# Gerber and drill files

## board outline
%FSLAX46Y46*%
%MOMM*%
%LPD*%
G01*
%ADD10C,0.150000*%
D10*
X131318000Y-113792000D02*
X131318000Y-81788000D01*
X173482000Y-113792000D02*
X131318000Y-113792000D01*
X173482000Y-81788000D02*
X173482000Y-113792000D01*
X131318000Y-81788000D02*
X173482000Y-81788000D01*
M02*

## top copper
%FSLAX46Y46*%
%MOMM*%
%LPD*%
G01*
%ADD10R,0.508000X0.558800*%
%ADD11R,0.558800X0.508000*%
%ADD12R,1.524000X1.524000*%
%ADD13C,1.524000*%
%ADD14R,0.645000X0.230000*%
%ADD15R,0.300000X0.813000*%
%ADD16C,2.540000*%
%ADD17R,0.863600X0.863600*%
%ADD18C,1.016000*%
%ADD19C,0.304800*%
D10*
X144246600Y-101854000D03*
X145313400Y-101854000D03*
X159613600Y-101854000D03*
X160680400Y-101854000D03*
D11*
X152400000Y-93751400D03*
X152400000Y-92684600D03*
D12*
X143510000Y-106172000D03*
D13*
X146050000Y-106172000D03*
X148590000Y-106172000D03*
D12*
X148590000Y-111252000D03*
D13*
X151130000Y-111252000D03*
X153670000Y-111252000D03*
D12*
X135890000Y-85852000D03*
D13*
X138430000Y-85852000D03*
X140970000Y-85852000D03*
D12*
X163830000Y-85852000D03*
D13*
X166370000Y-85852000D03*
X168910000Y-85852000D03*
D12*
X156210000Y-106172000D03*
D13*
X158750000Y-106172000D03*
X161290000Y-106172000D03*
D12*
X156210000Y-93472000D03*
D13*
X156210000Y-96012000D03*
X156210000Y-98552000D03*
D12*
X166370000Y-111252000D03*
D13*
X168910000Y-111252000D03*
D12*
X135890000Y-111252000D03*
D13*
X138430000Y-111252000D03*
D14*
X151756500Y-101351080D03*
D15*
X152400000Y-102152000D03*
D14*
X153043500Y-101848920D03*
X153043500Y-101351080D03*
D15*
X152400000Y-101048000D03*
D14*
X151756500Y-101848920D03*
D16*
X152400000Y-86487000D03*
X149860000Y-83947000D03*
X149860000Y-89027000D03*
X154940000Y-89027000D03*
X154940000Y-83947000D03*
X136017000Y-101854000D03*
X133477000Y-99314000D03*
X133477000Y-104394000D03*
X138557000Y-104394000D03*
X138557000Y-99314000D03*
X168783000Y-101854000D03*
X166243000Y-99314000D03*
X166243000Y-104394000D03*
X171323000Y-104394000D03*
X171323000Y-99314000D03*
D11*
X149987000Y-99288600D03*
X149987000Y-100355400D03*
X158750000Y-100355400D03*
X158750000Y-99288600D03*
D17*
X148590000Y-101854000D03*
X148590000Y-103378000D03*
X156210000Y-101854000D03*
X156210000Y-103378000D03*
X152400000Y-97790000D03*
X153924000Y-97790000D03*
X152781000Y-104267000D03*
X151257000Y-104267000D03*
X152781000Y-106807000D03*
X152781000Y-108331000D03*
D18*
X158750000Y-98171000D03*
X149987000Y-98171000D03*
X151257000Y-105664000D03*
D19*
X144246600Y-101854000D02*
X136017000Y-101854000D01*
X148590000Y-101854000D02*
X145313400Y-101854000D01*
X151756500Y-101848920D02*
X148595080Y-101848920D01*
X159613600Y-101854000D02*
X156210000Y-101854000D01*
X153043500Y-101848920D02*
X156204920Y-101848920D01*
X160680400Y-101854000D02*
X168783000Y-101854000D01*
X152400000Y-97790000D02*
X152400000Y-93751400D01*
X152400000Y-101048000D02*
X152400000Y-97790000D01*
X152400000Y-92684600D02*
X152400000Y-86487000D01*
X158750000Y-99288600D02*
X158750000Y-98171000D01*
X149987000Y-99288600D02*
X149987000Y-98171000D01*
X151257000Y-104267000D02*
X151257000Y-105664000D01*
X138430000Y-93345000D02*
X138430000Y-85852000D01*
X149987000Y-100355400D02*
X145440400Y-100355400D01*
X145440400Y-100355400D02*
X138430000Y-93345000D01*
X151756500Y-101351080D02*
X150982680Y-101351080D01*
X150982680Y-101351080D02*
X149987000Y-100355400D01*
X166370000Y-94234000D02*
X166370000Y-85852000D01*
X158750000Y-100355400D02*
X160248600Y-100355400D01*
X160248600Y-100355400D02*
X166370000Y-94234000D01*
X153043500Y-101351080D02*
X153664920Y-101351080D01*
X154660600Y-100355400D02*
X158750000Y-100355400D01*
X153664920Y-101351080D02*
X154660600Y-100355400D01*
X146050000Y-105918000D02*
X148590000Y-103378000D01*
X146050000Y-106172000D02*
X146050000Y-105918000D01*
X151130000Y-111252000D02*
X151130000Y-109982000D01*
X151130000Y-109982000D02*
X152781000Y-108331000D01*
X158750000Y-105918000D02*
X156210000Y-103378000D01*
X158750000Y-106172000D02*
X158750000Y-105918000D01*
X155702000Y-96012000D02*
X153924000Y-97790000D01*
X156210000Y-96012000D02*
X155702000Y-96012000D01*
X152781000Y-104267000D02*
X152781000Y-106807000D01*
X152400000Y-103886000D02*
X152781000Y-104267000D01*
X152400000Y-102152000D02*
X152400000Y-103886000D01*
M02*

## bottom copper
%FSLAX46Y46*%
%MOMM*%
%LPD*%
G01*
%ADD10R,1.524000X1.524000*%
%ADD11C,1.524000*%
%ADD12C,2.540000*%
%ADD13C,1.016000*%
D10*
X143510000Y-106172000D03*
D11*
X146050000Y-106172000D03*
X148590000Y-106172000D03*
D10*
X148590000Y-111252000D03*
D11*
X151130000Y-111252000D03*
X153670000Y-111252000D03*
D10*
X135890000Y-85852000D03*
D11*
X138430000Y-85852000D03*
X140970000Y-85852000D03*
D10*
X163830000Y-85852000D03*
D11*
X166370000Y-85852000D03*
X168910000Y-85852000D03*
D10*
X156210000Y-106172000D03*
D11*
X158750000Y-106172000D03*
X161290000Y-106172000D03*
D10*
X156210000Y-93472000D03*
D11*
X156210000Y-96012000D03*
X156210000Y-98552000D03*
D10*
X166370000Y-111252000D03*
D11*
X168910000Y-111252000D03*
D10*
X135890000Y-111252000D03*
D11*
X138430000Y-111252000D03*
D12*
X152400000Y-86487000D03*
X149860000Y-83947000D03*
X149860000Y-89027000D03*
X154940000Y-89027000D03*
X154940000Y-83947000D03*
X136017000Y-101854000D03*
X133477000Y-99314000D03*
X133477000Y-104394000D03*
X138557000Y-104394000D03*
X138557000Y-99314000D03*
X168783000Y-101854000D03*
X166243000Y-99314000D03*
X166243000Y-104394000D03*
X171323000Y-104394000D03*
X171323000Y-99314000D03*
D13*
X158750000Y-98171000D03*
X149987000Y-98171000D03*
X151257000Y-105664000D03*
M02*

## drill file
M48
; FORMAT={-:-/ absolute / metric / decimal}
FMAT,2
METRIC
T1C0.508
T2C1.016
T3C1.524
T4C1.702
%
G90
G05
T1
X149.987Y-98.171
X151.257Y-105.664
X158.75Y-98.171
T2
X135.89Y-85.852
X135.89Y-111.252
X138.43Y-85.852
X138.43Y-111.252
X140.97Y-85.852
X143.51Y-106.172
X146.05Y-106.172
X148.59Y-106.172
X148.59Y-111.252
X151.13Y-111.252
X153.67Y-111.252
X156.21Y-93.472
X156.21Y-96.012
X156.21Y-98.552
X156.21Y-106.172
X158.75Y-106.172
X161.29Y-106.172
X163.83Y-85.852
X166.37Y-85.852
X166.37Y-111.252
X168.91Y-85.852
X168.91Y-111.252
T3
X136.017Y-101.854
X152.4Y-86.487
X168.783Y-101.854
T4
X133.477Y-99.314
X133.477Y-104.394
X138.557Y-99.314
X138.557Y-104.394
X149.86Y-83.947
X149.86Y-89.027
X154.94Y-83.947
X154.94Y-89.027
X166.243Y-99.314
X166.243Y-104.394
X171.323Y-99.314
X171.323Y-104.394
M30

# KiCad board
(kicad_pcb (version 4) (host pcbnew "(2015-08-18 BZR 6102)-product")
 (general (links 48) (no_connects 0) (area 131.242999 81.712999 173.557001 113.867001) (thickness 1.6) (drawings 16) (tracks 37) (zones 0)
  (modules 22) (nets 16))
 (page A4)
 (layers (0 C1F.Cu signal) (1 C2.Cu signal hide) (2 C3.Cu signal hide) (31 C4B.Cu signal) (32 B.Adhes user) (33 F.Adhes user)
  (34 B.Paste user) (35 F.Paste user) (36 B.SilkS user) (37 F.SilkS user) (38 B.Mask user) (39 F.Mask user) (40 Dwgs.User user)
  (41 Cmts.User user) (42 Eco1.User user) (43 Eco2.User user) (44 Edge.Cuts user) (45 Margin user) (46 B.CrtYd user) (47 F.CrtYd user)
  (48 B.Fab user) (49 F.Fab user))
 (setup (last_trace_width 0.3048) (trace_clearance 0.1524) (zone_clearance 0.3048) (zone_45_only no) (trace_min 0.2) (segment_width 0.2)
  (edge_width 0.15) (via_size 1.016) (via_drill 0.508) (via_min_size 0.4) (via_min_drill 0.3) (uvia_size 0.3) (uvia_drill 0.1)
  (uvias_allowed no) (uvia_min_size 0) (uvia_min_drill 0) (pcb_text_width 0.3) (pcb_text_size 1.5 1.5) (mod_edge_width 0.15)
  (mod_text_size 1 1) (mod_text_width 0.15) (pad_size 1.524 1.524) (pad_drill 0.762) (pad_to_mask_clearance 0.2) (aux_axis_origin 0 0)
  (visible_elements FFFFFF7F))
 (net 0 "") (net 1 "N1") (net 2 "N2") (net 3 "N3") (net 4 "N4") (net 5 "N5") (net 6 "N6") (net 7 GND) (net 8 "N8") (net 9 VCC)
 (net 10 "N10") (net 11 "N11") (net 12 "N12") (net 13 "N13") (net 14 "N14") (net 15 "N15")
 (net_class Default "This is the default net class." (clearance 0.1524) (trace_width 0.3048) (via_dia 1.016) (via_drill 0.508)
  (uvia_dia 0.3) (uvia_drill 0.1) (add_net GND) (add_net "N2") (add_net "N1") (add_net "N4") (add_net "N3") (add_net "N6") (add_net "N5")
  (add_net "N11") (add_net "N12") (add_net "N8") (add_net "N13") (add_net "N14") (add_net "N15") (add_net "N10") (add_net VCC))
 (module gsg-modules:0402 (layer C1F.Cu) (at 144.78 101.854 180) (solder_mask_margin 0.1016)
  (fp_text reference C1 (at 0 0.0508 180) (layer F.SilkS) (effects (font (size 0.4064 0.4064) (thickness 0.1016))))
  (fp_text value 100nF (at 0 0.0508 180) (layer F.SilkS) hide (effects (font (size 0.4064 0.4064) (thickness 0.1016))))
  (pad 2 smd rect (at 0.5334 0 180) (size 0.508 0.5588) (layers C1F.Cu F.Paste F.Mask) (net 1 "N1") (solder_mask_margin 0.1016))
  (pad 1 smd rect (at -0.5334 0 180) (size 0.508 0.5588) (layers C1F.Cu F.Paste F.Mask) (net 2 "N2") (solder_mask_margin 0.1016)))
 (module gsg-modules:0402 (layer C1F.Cu) (at 160.147 101.854 180) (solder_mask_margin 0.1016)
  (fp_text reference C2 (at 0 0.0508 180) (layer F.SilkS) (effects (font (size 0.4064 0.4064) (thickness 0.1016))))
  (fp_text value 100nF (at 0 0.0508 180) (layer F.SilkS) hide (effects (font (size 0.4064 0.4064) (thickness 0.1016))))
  (pad 2 smd rect (at 0.5334 0 180) (size 0.508 0.5588) (layers C1F.Cu F.Paste F.Mask) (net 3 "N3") (solder_mask_margin 0.1016))
  (pad 1 smd rect (at -0.5334 0 180) (size 0.508 0.5588) (layers C1F.Cu F.Paste F.Mask) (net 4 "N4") (solder_mask_margin 0.1016)))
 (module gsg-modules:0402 (layer C1F.Cu) (at 152.4 93.218 270) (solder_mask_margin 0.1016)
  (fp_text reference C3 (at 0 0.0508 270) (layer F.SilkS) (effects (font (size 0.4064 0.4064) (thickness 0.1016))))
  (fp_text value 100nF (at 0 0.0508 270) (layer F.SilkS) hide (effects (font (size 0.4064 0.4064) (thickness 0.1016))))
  (pad 2 smd rect (at 0.5334 0 270) (size 0.508 0.5588) (layers C1F.Cu F.Paste F.Mask) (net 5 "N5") (solder_mask_margin 0.1016))
  (pad 1 smd rect (at -0.5334 0 270) (size 0.508 0.5588) (layers C1F.Cu F.Paste F.Mask) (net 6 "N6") (solder_mask_margin 0.1016)))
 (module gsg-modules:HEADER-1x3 (layer C1F.Cu) (at 146.05 106.172)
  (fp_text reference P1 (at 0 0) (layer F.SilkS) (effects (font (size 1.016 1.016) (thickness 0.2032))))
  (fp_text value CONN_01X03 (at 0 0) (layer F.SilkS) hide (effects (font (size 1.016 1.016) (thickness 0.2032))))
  (pad 1 thru_hole rect (at -2.54 0) (size 1.524 1.524) (drill 1.016) (layers *.Cu *.Mask F.SilkS) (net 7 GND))
  (pad 2 thru_hole circle (at 0 0) (size 1.524 1.524) (drill 1.016) (layers *.Cu *.Mask F.SilkS) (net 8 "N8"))
  (pad 3 thru_hole circle (at 2.54 0) (size 1.524 1.524) (drill 1.016) (layers *.Cu *.Mask F.SilkS) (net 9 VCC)))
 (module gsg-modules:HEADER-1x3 (layer C1F.Cu) (at 151.13 111.252)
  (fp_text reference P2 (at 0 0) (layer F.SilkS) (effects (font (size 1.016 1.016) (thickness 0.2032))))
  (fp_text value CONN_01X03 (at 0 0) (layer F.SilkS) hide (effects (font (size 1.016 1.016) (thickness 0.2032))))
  (pad 1 thru_hole rect (at -2.54 0) (size 1.524 1.524) (drill 1.016) (layers *.Cu *.Mask F.SilkS) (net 7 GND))
  (pad 2 thru_hole circle (at 0 0) (size 1.524 1.524) (drill 1.016) (layers *.Cu *.Mask F.SilkS) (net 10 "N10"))
  (pad 3 thru_hole circle (at 2.54 0) (size 1.524 1.524) (drill 1.016) (layers *.Cu *.Mask F.SilkS) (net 9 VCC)))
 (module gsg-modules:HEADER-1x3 (layer C1F.Cu) (at 138.43 85.852)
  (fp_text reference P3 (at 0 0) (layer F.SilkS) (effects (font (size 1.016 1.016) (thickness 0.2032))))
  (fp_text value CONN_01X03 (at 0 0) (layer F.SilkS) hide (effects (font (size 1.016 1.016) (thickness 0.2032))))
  (pad 1 thru_hole rect (at -2.54 0) (size 1.524 1.524) (drill 1.016) (layers *.Cu *.Mask F.SilkS) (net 7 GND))
  (pad 2 thru_hole circle (at 0 0) (size 1.524 1.524) (drill 1.016) (layers *.Cu *.Mask F.SilkS) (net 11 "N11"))
  (pad 3 thru_hole circle (at 2.54 0) (size 1.524 1.524) (drill 1.016) (layers *.Cu *.Mask F.SilkS) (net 9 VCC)))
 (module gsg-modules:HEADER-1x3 (layer C1F.Cu) (at 166.37 85.852)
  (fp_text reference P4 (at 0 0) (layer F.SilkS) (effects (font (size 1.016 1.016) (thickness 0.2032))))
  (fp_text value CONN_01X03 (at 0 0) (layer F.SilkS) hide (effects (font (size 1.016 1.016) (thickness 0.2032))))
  (pad 1 thru_hole rect (at -2.54 0) (size 1.524 1.524) (drill 1.016) (layers *.Cu *.Mask F.SilkS) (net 7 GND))
  (pad 2 thru_hole circle (at 0 0) (size 1.524 1.524) (drill 1.016) (layers *.Cu *.Mask F.SilkS) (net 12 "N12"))
  (pad 3 thru_hole circle (at 2.54 0) (size 1.524 1.524) (drill 1.016) (layers *.Cu *.Mask F.SilkS) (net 9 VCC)))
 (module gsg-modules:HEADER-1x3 (layer C1F.Cu) (at 158.75 106.172)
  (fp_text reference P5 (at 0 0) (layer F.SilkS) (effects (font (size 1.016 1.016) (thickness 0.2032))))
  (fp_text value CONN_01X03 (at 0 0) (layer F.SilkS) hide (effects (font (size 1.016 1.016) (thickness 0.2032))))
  (pad 1 thru_hole rect (at -2.54 0) (size 1.524 1.524) (drill 1.016) (layers *.Cu *.Mask F.SilkS) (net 7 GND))
  (pad 2 thru_hole circle (at 0 0) (size 1.524 1.524) (drill 1.016) (layers *.Cu *.Mask F.SilkS) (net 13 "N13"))
  (pad 3 thru_hole circle (at 2.54 0) (size 1.524 1.524) (drill 1.016) (layers *.Cu *.Mask F.SilkS) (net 9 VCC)))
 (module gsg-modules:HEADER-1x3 (layer C1F.Cu) (at 156.21 96.012 270)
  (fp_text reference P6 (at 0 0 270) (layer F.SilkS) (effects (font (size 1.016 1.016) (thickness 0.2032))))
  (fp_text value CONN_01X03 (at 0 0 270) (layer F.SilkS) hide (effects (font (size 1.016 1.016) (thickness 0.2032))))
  (pad 1 thru_hole rect (at -2.54 0 270) (size 1.524 1.524) (drill 1.016) (layers *.Cu *.Mask F.SilkS) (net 7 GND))
  (pad 2 thru_hole circle (at 0 0 270) (size 1.524 1.524) (drill 1.016) (layers *.Cu *.Mask F.SilkS) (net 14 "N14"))
  (pad 3 thru_hole circle (at 2.54 0 270) (size 1.524 1.524) (drill 1.016) (layers *.Cu *.Mask F.SilkS) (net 9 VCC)))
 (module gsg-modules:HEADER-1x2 (layer C1F.Cu) (at 167.64 111.252)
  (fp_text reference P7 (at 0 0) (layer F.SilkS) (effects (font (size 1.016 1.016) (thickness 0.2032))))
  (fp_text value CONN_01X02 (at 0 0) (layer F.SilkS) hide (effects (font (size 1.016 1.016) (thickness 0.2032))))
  (pad 1 thru_hole rect (at -1.27 0) (size 1.524 1.524) (drill 1.016) (layers *.Cu *.Mask F.SilkS) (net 9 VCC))
  (pad 2 thru_hole circle (at 1.27 0) (size 1.524 1.524) (drill 1.016) (layers *.Cu *.Mask F.SilkS) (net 9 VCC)))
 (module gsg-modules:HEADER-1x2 (layer C1F.Cu) (at 137.16 111.252)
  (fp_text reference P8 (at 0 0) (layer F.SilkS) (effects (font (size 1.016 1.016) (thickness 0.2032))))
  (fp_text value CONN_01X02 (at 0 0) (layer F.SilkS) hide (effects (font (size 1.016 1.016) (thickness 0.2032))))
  (pad 1 thru_hole rect (at -1.27 0) (size 1.524 1.524) (drill 1.016) (layers *.Cu *.Mask F.SilkS) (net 7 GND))
  (pad 2 thru_hole circle (at 1.27 0) (size 1.524 1.524) (drill 1.016) (layers *.Cu *.Mask F.SilkS) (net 7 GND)))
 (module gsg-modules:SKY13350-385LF (layer C1F.Cu) (at 152.4 101.6) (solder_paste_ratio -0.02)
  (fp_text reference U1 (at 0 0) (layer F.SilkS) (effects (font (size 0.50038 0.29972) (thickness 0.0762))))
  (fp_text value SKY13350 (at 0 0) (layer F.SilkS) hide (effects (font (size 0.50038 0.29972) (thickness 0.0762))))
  (pad 1 smd rect (at -0.6435 -0.24892) (size 0.645 0.23) (layers C1F.Cu F.Paste F.Mask) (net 11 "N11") (die_length -2147.483648))
  (pad 3 smd rect (at 0 0.552) (size 0.3 0.813) (layers C1F.Cu F.Paste F.Mask) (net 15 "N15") (die_length -2147.483648))
  (pad 4 smd rect (at 0.6435 0.24892) (size 0.645 0.23) (layers C1F.Cu F.Paste F.Mask) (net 3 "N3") (die_length 0.0508))
  (pad 5 smd rect (at 0.6435 -0.24892) (size 0.645 0.23) (layers C1F.Cu F.Paste F.Mask) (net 12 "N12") (die_length 10.53846))
  (pad 6 smd rect (at 0 -0.552) (size 0.3 0.813) (layers C1F.Cu F.Paste F.Mask) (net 5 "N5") (die_length -2147.483648))
  (pad 2 smd rect (at -0.6435 0.24892) (size 0.645 0.23) (layers C1F.Cu F.Paste F.Mask) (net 2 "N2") (die_length -2147.483648)))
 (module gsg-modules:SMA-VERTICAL (layer C1F.Cu) (at 152.4 86.487)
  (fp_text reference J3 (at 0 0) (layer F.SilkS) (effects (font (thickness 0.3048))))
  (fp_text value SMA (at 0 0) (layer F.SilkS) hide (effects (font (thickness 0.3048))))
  (pad 1 thru_hole circle (at 0 0) (size 2.54 2.54) (drill 1.524) (layers *.Cu *.Mask F.SilkS) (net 6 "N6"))
  (pad 2 thru_hole circle (at -2.54 -2.54) (size 2.54 2.54) (drill 1.7018) (layers *.Cu *.Mask F.SilkS) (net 7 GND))
  (pad 2 thru_hole circle (at -2.54 2.54) (size 2.54 2.54) (drill 1.7018) (layers *.Cu *.Mask F.SilkS) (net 7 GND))
  (pad 2 thru_hole circle (at 2.54 2.54) (size 2.54 2.54) (drill 1.7018) (layers *.Cu *.Mask F.SilkS) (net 7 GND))
  (pad 2 thru_hole circle (at 2.54 -2.54) (size 2.54 2.54) (drill 1.7018) (layers *.Cu *.Mask F.SilkS) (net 7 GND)))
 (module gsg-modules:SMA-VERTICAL (layer C1F.Cu) (at 136.017 101.854)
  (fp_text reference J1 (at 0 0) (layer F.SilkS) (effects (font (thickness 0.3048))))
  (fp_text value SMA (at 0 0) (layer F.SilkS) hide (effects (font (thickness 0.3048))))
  (pad 1 thru_hole circle (at 0 0) (size 2.54 2.54) (drill 1.524) (layers *.Cu *.Mask F.SilkS) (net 1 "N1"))
  (pad 2 thru_hole circle (at -2.54 -2.54) (size 2.54 2.54) (drill 1.7018) (layers *.Cu *.Mask F.SilkS) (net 7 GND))
  (pad 2 thru_hole circle (at -2.54 2.54) (size 2.54 2.54) (drill 1.7018) (layers *.Cu *.Mask F.SilkS) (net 7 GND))
  (pad 2 thru_hole circle (at 2.54 2.54) (size 2.54 2.54) (drill 1.7018) (layers *.Cu *.Mask F.SilkS) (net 7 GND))
  (pad 2 thru_hole circle (at 2.54 -2.54) (size 2.54 2.54) (drill 1.7018) (layers *.Cu *.Mask F.SilkS) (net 7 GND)))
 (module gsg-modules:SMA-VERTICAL (layer C1F.Cu) (at 168.783 101.854)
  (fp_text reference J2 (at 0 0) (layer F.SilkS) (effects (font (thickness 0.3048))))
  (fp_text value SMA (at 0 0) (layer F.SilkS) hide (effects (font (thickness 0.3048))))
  (pad 1 thru_hole circle (at 0 0) (size 2.54 2.54) (drill 1.524) (layers *.Cu *.Mask F.SilkS) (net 4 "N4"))
  (pad 2 thru_hole circle (at -2.54 -2.54) (size 2.54 2.54) (drill 1.7018) (layers *.Cu *.Mask F.SilkS) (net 7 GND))
  (pad 2 thru_hole circle (at -2.54 2.54) (size 2.54 2.54) (drill 1.7018) (layers *.Cu *.Mask F.SilkS) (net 7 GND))
  (pad 2 thru_hole circle (at 2.54 2.54) (size 2.54 2.54) (drill 1.7018) (layers *.Cu *.Mask F.SilkS) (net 7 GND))
  (pad 2 thru_hole circle (at 2.54 -2.54) (size 2.54 2.54) (drill 1.7018) (layers *.Cu *.Mask F.SilkS) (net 7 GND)))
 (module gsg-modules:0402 (layer C1F.Cu) (at 149.987 99.822 90) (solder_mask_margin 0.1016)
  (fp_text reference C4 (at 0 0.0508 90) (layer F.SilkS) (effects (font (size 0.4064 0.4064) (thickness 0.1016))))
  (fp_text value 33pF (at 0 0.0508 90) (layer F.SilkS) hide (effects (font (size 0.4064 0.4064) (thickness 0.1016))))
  (pad 2 smd rect (at 0.5334 0 90) (size 0.508 0.5588) (layers C1F.Cu F.Paste F.Mask) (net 7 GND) (solder_mask_margin 0.1016))
  (pad 1 smd rect (at -0.5334 0 90) (size 0.508 0.5588) (layers C1F.Cu F.Paste F.Mask) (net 11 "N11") (solder_mask_margin 0.1016)))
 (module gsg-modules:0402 (layer C1F.Cu) (at 158.75 99.822 270) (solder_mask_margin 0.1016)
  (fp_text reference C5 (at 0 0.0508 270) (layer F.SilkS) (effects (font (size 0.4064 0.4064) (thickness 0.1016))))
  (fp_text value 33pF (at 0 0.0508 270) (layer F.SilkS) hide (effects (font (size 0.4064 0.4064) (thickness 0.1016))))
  (pad 2 smd rect (at 0.5334 0 270) (size 0.508 0.5588) (layers C1F.Cu F.Paste F.Mask) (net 12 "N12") (solder_mask_margin 0.1016))
  (pad 1 smd rect (at -0.5334 0 270) (size 0.508 0.5588) (layers C1F.Cu F.Paste F.Mask) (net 7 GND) (solder_mask_margin 0.1016)))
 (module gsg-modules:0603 (layer C1F.Cu) (at 148.59 102.616 90) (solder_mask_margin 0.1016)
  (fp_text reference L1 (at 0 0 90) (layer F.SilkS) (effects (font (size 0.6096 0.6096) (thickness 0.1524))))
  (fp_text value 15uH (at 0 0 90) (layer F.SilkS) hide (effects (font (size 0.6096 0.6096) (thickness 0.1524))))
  (pad 2 smd rect (at 0.762 0 90) (size 0.8636 0.8636) (layers C1F.Cu F.Paste F.Mask) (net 2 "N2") (solder_mask_margin 0.1016)
   (clearance 0.1778))
  (pad 1 smd rect (at -0.762 0 90) (size 0.8636 0.8636) (layers C1F.Cu F.Paste F.Mask) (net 8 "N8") (solder_mask_margin 0.1016)
   (clearance 0.1778)))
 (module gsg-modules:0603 (layer C1F.Cu) (at 156.21 102.616 90) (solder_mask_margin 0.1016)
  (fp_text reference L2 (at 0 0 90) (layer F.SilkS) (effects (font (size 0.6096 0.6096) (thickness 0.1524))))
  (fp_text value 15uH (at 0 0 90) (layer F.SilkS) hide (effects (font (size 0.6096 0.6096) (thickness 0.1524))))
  (pad 2 smd rect (at 0.762 0 90) (size 0.8636 0.8636) (layers C1F.Cu F.Paste F.Mask) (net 3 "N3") (solder_mask_margin 0.1016)
   (clearance 0.1778))
  (pad 1 smd rect (at -0.762 0 90) (size 0.8636 0.8636) (layers C1F.Cu F.Paste F.Mask) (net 13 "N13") (solder_mask_margin 0.1016)
   (clearance 0.1778)))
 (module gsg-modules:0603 (layer C1F.Cu) (at 153.162 97.79 180) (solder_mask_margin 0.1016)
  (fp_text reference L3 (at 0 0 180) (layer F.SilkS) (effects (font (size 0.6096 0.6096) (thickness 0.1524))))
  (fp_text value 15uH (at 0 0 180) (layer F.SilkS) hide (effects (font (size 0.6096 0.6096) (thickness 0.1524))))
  (pad 2 smd rect (at 0.762 0 180) (size 0.8636 0.8636) (layers C1F.Cu F.Paste F.Mask) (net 5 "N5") (solder_mask_margin 0.1016)
   (clearance 0.1778))
  (pad 1 smd rect (at -0.762 0 180) (size 0.8636 0.8636) (layers C1F.Cu F.Paste F.Mask) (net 14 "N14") (solder_mask_margin 0.1016)
   (clearance 0.1778)))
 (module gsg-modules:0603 (layer C1F.Cu) (at 152.019 104.267) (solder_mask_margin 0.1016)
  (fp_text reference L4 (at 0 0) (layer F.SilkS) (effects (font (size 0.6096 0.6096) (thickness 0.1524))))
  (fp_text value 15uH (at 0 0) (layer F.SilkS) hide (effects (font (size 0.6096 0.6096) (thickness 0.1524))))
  (pad 2 smd rect (at 0.762 0) (size 0.8636 0.8636) (layers C1F.Cu F.Paste F.Mask) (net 15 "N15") (solder_mask_margin 0.1016)
   (clearance 0.1778))
  (pad 1 smd rect (at -0.762 0) (size 0.8636 0.8636) (layers C1F.Cu F.Paste F.Mask) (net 7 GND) (solder_mask_margin 0.1016)
   (clearance 0.1778)))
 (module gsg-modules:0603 (layer C1F.Cu) (at 152.781 107.569 90) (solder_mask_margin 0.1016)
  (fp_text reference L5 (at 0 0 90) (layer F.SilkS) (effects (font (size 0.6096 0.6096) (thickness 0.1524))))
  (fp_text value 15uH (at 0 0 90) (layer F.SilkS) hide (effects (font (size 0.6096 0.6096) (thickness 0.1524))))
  (pad 2 smd rect (at 0.762 0 90) (size 0.8636 0.8636) (layers C1F.Cu F.Paste F.Mask) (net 15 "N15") (solder_mask_margin 0.1016)
   (clearance 0.1778))
  (pad 1 smd rect (at -0.762 0 90) (size 0.8636 0.8636) (layers C1F.Cu F.Paste F.Mask) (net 10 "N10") (solder_mask_margin 0.1016)
   (clearance 0.1778)))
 (gr_line (start 131.318 113.792) (end 131.318 81.788) (angle 90) (layer Edge.Cuts) (width 0.15))
 (gr_line (start 173.482 113.792) (end 131.318 113.792) (angle 90) (layer Edge.Cuts) (width 0.15))
 (gr_line (start 173.482 81.788) (end 173.482 113.792) (angle 90) (layer Edge.Cuts) (width 0.15))
 (gr_line (start 131.318 81.788) (end 173.482 81.788) (angle 90) (layer Edge.Cuts) (width 0.15))
 (segment (start 144.2466 101.854) (end 136.017 101.854) (width 0.3048) (layer C1F.Cu) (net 1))
 (segment (start 148.59 101.854) (end 145.3134 101.854) (width 0.3048) (layer C1F.Cu) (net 2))
 (segment (start 151.7565 101.84892) (end 148.59508 101.84892) (width 0.3048) (layer C1F.Cu) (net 2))
 (segment (start 159.6136 101.854) (end 156.21 101.854) (width 0.3048) (layer C1F.Cu) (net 3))
 (segment (start 153.0435 101.84892) (end 156.20492 101.84892) (width 0.3048) (layer C1F.Cu) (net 3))
 (segment (start 160.6804 101.854) (end 168.783 101.854) (width 0.3048) (layer C1F.Cu) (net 4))
 (segment (start 152.4 97.79) (end 152.4 93.7514) (width 0.3048) (layer C1F.Cu) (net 5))
 (segment (start 152.4 101.048) (end 152.4 97.79) (width 0.3048) (layer C1F.Cu) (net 5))
 (segment (start 152.4 92.6846) (end 152.4 86.487) (width 0.3048) (layer C1F.Cu) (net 6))
 (segment (start 158.75 99.2886) (end 158.75 98.171) (width 0.3048) (layer C1F.Cu) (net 7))
 (via (at 158.75 98.171) (size 1.016) (drill 0.508) (layers C1F.Cu C4B.Cu) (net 7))
 (segment (start 149.987 99.2886) (end 149.987 98.171) (width 0.3048) (layer C1F.Cu) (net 7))
 (via (at 149.987 98.171) (size 1.016) (drill 0.508) (layers C1F.Cu C4B.Cu) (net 7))
 (segment (start 151.257 104.267) (end 151.257 105.664) (width 0.3048) (layer C1F.Cu) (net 7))
 (via (at 151.257 105.664) (size 1.016) (drill 0.508) (layers C1F.Cu C4B.Cu) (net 7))
 (segment (start 138.43 93.345) (end 138.43 85.852) (width 0.3048) (layer C1F.Cu) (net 11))
 (segment (start 149.987 100.3554) (end 145.4404 100.3554) (width 0.3048) (layer C1F.Cu) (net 11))
 (segment (start 145.4404 100.3554) (end 138.43 93.345) (width 0.3048) (layer C1F.Cu) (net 11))
 (segment (start 151.7565 101.35108) (end 150.98268 101.35108) (width 0.3048) (layer C1F.Cu) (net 11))
 (segment (start 150.98268 101.35108) (end 149.987 100.3554) (width 0.3048) (layer C1F.Cu) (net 11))
 (segment (start 166.37 94.234) (end 166.37 85.852) (width 0.3048) (layer C1F.Cu) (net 12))
 (segment (start 158.75 100.3554) (end 160.2486 100.3554) (width 0.3048) (layer C1F.Cu) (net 12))
 (segment (start 160.2486 100.3554) (end 166.37 94.234) (width 0.3048) (layer C1F.Cu) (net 12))
 (segment (start 153.0435 101.35108) (end 153.66492 101.35108) (width 0.3048) (layer C1F.Cu) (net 12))
 (segment (start 154.6606 100.3554) (end 158.75 100.3554) (width 0.3048) (layer C1F.Cu) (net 12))
 (segment (start 153.66492 101.35108) (end 154.6606 100.3554) (width 0.3048) (layer C1F.Cu) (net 12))
 (segment (start 146.05 105.918) (end 148.59 103.378) (width 0.3048) (layer C1F.Cu) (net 8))
 (segment (start 146.05 106.172) (end 146.05 105.918) (width 0.3048) (layer C1F.Cu) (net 8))
 (segment (start 151.13 111.252) (end 151.13 109.982) (width 0.3048) (layer C1F.Cu) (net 10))
 (segment (start 151.13 109.982) (end 152.781 108.331) (width 0.3048) (layer C1F.Cu) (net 10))
 (segment (start 158.75 105.918) (end 156.21 103.378) (width 0.3048) (layer C1F.Cu) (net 13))
 (segment (start 158.75 106.172) (end 158.75 105.918) (width 0.3048) (layer C1F.Cu) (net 13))
 (segment (start 155.702 96.012) (end 153.924 97.79) (width 0.3048) (layer C1F.Cu) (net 14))
 (segment (start 156.21 96.012) (end 155.702 96.012) (width 0.3048) (layer C1F.Cu) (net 14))
 (segment (start 152.781 104.267) (end 152.781 106.807) (width 0.3048) (layer C1F.Cu) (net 15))
 (segment (start 152.4 103.886) (end 152.781 104.267) (width 0.3048) (layer C1F.Cu) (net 15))
 (segment (start 152.4 102.152) (end 152.4 103.886) (width 0.3048) (layer C1F.Cu) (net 15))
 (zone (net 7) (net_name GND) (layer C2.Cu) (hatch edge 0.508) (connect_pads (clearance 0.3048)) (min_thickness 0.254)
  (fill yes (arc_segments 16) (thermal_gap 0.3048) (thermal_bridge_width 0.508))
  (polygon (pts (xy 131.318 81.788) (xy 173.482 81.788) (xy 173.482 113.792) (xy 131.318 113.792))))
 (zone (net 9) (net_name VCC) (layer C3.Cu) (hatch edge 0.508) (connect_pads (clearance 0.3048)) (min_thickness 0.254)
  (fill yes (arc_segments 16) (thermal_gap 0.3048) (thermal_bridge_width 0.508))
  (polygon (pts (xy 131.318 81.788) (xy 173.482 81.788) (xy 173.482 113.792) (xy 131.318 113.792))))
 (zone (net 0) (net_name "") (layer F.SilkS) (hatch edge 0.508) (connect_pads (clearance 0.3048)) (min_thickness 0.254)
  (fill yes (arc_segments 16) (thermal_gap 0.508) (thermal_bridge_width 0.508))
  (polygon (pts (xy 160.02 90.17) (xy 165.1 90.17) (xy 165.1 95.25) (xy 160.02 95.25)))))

